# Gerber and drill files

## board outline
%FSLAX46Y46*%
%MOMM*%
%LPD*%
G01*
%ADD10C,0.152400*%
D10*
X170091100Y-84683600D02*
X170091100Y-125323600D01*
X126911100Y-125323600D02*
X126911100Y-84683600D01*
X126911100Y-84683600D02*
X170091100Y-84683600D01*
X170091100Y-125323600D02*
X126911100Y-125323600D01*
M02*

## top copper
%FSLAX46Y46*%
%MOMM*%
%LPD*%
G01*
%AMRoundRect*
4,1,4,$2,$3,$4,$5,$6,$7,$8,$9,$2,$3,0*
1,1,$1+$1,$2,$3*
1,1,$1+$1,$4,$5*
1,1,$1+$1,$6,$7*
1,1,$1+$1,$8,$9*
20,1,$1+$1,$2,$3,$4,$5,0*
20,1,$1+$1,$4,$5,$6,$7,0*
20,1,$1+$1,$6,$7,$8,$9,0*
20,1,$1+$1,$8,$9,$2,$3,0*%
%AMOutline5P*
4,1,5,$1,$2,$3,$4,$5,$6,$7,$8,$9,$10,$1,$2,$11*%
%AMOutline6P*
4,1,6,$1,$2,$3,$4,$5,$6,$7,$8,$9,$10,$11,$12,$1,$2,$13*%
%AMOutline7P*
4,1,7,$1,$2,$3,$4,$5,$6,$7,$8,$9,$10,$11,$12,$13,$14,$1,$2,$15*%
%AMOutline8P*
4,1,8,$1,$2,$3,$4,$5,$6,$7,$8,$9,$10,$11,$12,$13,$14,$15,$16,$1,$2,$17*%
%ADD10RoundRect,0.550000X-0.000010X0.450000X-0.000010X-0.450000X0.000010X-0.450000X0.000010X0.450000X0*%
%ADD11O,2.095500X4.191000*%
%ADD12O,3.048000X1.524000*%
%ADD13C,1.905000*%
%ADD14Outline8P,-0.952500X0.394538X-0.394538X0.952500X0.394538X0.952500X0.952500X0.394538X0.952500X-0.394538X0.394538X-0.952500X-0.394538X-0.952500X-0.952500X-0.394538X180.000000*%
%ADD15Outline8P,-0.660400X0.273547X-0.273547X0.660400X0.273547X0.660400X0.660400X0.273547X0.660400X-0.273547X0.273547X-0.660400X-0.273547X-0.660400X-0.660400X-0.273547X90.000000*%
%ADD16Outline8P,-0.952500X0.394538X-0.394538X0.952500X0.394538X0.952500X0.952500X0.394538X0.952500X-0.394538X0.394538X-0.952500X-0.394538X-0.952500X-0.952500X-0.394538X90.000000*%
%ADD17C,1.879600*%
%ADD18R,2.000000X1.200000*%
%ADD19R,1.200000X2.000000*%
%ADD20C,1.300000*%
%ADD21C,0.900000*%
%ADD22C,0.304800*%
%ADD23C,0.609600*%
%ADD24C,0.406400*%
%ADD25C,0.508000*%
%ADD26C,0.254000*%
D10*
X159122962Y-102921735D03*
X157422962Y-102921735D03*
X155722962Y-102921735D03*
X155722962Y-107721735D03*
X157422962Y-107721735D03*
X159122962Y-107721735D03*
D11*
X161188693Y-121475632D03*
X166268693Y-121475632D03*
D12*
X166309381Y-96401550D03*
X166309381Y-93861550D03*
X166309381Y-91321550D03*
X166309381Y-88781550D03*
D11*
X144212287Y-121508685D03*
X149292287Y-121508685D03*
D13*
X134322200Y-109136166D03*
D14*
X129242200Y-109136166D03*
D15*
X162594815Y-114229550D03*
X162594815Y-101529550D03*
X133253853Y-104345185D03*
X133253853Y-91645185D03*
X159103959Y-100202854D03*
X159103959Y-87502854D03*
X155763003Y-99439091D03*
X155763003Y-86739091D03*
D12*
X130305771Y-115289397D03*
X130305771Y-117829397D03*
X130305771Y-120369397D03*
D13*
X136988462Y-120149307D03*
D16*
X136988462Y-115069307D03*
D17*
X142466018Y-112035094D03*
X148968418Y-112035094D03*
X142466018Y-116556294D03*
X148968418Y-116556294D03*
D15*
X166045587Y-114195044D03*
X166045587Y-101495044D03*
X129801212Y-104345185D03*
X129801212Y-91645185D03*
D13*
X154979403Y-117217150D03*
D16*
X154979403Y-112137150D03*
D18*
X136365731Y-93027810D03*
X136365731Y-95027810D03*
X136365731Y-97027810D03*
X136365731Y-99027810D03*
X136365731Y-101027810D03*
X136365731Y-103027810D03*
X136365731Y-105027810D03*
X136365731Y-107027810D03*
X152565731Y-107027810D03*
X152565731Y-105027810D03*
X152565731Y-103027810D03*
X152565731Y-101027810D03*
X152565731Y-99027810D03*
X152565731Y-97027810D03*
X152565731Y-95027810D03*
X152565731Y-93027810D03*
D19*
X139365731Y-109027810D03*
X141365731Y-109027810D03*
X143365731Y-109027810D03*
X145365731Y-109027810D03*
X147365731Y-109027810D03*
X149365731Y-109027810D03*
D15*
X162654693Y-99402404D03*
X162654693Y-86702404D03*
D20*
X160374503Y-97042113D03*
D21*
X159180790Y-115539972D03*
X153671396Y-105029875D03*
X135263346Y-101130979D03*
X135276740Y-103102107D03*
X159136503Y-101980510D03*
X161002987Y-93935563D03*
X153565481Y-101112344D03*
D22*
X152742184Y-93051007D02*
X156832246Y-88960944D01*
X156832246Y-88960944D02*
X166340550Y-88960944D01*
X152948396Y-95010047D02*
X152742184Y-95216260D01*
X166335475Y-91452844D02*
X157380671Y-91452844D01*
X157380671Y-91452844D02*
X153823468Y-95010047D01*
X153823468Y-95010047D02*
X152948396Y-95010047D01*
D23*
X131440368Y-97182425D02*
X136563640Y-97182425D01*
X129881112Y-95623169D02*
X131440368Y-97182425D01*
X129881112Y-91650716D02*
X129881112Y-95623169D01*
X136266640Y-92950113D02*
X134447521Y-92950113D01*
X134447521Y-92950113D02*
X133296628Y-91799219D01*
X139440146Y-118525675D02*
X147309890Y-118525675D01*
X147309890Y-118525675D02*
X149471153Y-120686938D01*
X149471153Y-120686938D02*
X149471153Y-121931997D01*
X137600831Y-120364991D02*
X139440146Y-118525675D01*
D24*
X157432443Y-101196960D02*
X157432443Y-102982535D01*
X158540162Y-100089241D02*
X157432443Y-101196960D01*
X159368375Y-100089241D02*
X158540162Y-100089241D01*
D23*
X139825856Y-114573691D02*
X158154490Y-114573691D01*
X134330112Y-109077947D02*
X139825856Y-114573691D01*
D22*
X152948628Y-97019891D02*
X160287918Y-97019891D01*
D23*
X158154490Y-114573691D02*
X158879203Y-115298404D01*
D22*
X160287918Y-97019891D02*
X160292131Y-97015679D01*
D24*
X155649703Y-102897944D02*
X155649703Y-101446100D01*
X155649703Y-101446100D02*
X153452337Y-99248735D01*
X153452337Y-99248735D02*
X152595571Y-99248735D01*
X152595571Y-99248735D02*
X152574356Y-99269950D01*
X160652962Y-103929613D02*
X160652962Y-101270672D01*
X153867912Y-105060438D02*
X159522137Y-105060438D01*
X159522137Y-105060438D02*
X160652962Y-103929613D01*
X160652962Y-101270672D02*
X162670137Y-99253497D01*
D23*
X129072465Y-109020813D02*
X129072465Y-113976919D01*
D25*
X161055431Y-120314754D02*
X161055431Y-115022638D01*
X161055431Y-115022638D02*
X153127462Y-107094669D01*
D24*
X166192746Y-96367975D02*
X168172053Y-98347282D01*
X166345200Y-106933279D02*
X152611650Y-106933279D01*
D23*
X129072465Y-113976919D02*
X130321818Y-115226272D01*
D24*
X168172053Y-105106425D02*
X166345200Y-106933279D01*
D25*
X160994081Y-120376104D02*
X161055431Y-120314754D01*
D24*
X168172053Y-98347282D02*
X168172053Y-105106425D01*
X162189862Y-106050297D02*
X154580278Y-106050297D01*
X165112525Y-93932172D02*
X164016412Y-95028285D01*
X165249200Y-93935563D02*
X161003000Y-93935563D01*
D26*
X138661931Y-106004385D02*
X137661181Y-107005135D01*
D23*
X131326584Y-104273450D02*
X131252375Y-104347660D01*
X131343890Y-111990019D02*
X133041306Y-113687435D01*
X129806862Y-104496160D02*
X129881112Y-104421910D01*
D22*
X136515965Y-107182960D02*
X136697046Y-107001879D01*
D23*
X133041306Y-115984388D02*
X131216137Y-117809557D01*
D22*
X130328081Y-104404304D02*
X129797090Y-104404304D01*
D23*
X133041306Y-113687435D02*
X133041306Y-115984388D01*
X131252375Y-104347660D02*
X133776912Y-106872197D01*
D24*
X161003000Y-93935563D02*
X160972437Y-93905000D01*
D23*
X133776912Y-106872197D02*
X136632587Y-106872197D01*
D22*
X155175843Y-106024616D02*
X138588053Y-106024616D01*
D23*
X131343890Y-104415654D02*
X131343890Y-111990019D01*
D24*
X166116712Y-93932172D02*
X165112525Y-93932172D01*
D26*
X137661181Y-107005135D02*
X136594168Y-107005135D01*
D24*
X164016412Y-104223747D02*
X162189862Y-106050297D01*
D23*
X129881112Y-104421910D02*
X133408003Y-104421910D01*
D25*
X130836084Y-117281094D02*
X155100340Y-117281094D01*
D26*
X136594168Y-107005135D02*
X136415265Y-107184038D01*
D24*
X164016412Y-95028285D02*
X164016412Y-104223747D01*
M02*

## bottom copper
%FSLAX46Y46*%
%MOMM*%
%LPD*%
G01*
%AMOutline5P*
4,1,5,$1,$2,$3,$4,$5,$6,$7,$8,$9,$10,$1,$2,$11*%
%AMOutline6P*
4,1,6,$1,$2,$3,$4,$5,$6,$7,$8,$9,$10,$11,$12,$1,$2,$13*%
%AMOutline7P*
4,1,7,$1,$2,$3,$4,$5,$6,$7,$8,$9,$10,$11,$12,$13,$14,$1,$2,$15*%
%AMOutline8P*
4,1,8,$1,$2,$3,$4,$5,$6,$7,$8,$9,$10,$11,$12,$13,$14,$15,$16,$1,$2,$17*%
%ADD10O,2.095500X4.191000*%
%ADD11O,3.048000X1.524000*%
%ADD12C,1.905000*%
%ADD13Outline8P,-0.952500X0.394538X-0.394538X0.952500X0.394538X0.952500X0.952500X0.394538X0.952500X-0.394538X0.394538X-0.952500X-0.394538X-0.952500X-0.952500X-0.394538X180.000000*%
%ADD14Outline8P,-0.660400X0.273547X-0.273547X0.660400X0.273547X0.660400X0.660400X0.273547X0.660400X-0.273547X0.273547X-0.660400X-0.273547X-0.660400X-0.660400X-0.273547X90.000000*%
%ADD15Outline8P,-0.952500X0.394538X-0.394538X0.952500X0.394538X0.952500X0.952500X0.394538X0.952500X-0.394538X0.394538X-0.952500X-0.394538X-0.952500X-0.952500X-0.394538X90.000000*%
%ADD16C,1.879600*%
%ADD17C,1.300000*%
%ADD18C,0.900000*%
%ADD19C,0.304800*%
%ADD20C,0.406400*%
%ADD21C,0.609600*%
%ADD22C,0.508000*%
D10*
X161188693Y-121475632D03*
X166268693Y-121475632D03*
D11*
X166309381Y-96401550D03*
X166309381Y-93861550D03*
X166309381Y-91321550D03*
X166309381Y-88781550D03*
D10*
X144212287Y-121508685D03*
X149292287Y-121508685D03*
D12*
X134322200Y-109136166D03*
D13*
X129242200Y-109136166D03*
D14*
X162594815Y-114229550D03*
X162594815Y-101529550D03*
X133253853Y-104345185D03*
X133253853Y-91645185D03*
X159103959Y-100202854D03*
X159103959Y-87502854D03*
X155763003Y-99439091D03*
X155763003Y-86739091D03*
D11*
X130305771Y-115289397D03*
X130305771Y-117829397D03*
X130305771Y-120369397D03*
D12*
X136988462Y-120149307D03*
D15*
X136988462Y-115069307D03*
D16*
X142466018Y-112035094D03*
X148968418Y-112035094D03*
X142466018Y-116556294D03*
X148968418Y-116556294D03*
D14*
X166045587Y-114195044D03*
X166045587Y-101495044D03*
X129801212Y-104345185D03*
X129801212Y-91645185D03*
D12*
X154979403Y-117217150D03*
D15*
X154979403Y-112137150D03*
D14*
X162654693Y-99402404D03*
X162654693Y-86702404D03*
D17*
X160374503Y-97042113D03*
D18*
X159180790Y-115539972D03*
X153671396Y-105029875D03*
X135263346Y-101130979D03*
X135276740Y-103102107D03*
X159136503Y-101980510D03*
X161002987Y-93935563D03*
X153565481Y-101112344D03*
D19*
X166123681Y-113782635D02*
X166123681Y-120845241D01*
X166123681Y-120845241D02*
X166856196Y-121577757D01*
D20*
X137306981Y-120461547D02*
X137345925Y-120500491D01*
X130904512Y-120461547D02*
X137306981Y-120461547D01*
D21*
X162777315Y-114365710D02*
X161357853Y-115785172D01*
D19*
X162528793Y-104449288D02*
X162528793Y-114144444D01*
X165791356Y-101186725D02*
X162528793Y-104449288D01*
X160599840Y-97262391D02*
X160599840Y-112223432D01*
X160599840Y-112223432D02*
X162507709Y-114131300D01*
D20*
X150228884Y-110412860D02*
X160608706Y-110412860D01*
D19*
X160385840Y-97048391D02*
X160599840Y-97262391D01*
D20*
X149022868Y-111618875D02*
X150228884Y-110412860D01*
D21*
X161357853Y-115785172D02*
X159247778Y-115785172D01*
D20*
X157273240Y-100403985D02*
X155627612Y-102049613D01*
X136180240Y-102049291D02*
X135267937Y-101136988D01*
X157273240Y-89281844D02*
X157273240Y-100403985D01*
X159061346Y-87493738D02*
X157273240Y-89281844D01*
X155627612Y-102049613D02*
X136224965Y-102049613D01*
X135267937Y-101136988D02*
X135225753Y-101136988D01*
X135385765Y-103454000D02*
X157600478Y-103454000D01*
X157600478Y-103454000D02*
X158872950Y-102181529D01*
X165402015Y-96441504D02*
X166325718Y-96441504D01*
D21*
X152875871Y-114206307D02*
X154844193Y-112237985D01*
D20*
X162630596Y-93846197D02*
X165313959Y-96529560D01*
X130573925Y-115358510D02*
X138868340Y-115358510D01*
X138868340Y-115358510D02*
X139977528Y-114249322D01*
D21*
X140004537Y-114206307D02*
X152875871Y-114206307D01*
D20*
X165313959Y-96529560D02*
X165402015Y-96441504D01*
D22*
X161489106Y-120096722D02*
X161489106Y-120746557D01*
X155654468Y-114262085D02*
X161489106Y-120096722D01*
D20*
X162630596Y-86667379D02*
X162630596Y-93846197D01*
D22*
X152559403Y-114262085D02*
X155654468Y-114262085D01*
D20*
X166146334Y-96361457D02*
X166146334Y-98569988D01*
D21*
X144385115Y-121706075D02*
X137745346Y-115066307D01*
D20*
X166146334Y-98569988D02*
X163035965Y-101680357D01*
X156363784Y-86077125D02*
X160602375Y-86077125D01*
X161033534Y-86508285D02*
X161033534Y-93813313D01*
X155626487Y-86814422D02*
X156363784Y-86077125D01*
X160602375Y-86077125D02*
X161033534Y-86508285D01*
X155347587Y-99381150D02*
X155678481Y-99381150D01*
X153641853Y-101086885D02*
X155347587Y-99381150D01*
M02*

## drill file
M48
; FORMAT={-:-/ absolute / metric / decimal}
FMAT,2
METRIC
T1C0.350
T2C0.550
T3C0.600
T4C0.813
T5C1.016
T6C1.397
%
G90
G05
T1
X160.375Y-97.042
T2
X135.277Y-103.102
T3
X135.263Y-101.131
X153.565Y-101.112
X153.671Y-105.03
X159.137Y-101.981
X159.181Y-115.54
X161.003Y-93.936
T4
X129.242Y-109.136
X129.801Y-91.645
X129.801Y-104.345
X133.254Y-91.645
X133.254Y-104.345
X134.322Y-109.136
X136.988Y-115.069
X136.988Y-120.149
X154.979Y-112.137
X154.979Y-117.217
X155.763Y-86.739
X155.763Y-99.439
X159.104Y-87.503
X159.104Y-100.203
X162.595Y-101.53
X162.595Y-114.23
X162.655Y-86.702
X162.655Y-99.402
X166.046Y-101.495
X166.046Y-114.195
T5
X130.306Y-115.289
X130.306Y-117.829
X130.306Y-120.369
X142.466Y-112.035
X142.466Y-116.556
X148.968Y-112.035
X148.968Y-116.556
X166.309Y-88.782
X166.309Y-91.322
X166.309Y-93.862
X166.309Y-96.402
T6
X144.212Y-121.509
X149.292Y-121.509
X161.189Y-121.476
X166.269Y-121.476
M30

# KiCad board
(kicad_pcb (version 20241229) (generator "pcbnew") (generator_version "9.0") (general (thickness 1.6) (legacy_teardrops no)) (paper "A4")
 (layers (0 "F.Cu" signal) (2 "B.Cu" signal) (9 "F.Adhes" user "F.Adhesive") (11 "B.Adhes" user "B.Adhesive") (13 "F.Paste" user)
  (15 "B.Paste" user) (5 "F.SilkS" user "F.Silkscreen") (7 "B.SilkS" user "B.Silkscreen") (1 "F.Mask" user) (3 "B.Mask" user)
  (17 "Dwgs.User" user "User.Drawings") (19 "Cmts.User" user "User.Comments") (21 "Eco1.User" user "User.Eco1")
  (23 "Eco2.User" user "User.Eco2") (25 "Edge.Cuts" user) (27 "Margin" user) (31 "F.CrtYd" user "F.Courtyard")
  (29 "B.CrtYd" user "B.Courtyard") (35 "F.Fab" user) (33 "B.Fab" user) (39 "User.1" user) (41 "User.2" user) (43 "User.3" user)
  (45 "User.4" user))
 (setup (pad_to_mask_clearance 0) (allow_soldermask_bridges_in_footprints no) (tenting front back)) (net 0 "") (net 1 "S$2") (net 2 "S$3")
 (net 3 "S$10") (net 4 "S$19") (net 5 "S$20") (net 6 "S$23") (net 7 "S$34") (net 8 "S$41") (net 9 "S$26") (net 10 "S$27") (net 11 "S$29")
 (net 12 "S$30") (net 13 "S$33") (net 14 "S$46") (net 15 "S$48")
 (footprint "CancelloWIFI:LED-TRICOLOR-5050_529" (layer "F.Cu") (at 157.422962 105.321735 -90)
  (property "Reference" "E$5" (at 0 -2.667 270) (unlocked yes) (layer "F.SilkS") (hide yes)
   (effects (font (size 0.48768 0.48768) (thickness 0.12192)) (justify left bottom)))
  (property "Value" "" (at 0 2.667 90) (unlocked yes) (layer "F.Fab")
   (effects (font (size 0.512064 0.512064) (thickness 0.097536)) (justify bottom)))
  (pad "1" smd roundrect (at -2.4 -1.7 270) (size 2 1.1) (layers "F.Cu" "F.Mask" "F.Paste") (roundrect_rratio 0.5)
   (solder_mask_margin 0.1016) (solder_paste_margin 0) (thermal_bridge_angle 0))
  (pad "2" smd roundrect (at -2.4 0 270) (size 2 1.1) (layers "F.Cu" "F.Mask" "F.Paste") (roundrect_rratio 0.5) (solder_mask_margin 0.1016)
   (solder_paste_margin 0) (thermal_bridge_angle 0))
  (pad "3" smd roundrect (at -2.4 1.7 270) (size 2 1.1) (layers "F.Cu" "F.Mask" "F.Paste") (roundrect_rratio 0.5)
   (solder_mask_margin 0.1016) (solder_paste_margin 0) (thermal_bridge_angle 0))
  (pad "4" smd roundrect (at 2.4 1.7 270) (size 2 1.1) (layers "F.Cu" "F.Mask" "F.Paste") (roundrect_rratio 0.5) (solder_mask_margin 0.1016)
   (solder_paste_margin 0) (thermal_bridge_angle 0))
  (pad "5" smd roundrect (at 2.4 0 270) (size 2 1.1) (layers "F.Cu" "F.Mask" "F.Paste") (roundrect_rratio 0.5) (solder_mask_margin 0.1016)
   (solder_paste_margin 0) (thermal_bridge_angle 0))
  (pad "6" smd roundrect (at 2.4 -1.7 270) (size 2 1.1) (layers "F.Cu" "F.Mask" "F.Paste") (roundrect_rratio 0.5)
   (solder_mask_margin 0.1016) (solder_paste_margin 0) (thermal_bridge_angle 0)))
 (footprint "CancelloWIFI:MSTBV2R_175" (layer "F.Cu") (at 163.728693 121.475632)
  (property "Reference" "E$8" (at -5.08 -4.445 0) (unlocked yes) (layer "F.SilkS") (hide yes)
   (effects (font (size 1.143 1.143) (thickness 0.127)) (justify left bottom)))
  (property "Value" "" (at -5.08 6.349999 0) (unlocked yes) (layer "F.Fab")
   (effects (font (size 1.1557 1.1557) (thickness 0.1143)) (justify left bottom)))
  (pad "1" thru_hole oval (at -2.54 0 90) (size 4.191 2.0955) (drill 1.397) (layers "*.Cu" "*.Mask") (remove_unused_layers no)
   (solder_mask_margin 0.1016) (thermal_bridge_angle 0))
  (pad "2" thru_hole oval (at 2.54 0 90) (size 4.191 2.0955) (drill 1.397) (layers "*.Cu" "*.Mask") (remove_unused_layers no)
   (solder_mask_margin 0.1016) (thermal_bridge_angle 0)))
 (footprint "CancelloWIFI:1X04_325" (layer "F.Cu") (at 166.309381 92.59155 90)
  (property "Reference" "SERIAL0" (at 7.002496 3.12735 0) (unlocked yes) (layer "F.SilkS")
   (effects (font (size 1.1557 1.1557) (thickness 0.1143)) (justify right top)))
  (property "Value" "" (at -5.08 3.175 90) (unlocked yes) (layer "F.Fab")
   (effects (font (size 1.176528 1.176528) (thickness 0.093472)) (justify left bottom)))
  (pad "1" thru_hole oval (at -3.81 0 180) (size 3.048 1.524) (drill 1.016) (layers "*.Cu" "*.Mask") (remove_unused_layers no)
   (solder_mask_margin 0.1016) (thermal_bridge_angle 0))
  (pad "2" thru_hole oval (at -1.27 0 180) (size 3.048 1.524) (drill 1.016) (layers "*.Cu" "*.Mask") (remove_unused_layers no)
   (solder_mask_margin 0.1016) (thermal_bridge_angle 0))
  (pad "3" thru_hole oval (at 1.27 0 180) (size 3.048 1.524) (drill 1.016) (layers "*.Cu" "*.Mask") (remove_unused_layers no)
   (solder_mask_margin 0.1016) (thermal_bridge_angle 0))
  (pad "4" thru_hole oval (at 3.81 0 180) (size 3.048 1.524) (drill 1.016) (layers "*.Cu" "*.Mask") (remove_unused_layers no)
   (solder_mask_margin 0.1016) (thermal_bridge_angle 0)))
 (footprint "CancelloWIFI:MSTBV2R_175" (layer "F.Cu") (at 146.752287 121.508685)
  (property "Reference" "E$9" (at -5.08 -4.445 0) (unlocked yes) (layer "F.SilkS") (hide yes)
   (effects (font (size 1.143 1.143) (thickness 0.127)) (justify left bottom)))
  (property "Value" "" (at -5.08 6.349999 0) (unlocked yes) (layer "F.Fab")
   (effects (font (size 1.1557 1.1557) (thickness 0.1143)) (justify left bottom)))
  (pad "1" thru_hole oval (at -2.54 0 90) (size 4.191 2.0955) (drill 1.397) (layers "*.Cu" "*.Mask") (remove_unused_layers no)
   (solder_mask_margin 0.1016) (thermal_bridge_angle 0))
  (pad "2" thru_hole oval (at 2.54 0 90) (size 4.191 2.0955) (drill 1.397) (layers "*.Cu" "*.Mask") (remove_unused_layers no)
   (solder_mask_margin 0.1016) (thermal_bridge_angle 0)))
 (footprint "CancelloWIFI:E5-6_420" (layer "F.Cu") (at 131.7822 109.136166 180)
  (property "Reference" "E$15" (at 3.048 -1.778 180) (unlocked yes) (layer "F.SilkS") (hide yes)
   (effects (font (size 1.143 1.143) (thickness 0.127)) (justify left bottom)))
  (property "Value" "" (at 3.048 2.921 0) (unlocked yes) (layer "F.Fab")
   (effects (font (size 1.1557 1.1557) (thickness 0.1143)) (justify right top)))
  (pad "+" thru_hole circle (at -2.54 0 180) (size 1.905 1.905) (drill 0.8128) (layers "*.Cu" "*.Mask") (remove_unused_layers no)
   (solder_mask_margin 0.1016) (thermal_bridge_angle 0))
  (pad "-" thru_hole roundrect (at 2.54 0 180) (size 1.905 1.905) (drill 0.8128) (layers "*.Cu" "*.Mask") (remove_unused_layers no)
   (roundrect_rratio 0.25) (chamfer_ratio 0.2928932188) (chamfer top_left top_right bottom_left bottom_right) (solder_mask_margin 0.1016)
   (thermal_bridge_angle 0)))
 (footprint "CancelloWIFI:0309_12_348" (layer "F.Cu") (at 162.594815 107.87955 90)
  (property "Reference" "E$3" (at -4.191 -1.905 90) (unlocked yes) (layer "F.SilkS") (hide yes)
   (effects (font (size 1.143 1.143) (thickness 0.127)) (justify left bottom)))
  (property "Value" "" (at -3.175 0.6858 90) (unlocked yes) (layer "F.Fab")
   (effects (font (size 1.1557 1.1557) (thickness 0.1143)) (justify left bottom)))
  (pad "1" thru_hole roundrect (at -6.35 0 90) (size 1.3208 1.3208) (drill 0.8128) (layers "*.Cu" "*.Mask") (remove_unused_layers no)
   (roundrect_rratio 0.25) (chamfer_ratio 0.2928932188) (chamfer top_left top_right bottom_left bottom_right) (solder_mask_margin 0.1016)
   (thermal_bridge_angle 0))
  (pad "2" thru_hole roundrect (at 6.35 0 90) (size 1.3208 1.3208) (drill 0.8128) (layers "*.Cu" "*.Mask") (remove_unused_layers no)
   (roundrect_rratio 0.25) (chamfer_ratio 0.2928932188) (chamfer top_left top_right bottom_left bottom_right) (solder_mask_margin 0.1016)
   (thermal_bridge_angle 0)))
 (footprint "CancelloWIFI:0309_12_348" (layer "F.Cu") (at 133.253853 97.995185 90)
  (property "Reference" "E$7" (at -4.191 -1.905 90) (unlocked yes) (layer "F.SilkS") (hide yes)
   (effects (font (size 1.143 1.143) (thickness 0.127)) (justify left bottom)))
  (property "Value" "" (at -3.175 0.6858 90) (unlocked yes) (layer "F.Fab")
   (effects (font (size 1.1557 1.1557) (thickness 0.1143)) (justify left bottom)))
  (pad "1" thru_hole roundrect (at -6.35 0 90) (size 1.3208 1.3208) (drill 0.8128) (layers "*.Cu" "*.Mask") (remove_unused_layers no)
   (roundrect_rratio 0.25) (chamfer_ratio 0.2928932188) (chamfer top_left top_right bottom_left bottom_right) (solder_mask_margin 0.1016)
   (thermal_bridge_angle 0))
  (pad "2" thru_hole roundrect (at 6.35 0 90) (size 1.3208 1.3208) (drill 0.8128) (layers "*.Cu" "*.Mask") (remove_unused_layers no)
   (roundrect_rratio 0.25) (chamfer_ratio 0.2928932188) (chamfer top_left top_right bottom_left bottom_right) (solder_mask_margin 0.1016)
   (thermal_bridge_angle 0)))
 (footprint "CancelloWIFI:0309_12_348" (layer "F.Cu") (at 159.103959 93.852854 90)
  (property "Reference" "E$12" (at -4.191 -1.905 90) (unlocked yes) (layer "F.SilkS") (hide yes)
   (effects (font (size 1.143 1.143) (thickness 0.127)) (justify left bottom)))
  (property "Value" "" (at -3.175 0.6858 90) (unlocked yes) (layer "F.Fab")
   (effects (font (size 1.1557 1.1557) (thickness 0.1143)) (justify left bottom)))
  (pad "1" thru_hole roundrect (at -6.35 0 90) (size 1.3208 1.3208) (drill 0.8128) (layers "*.Cu" "*.Mask") (remove_unused_layers no)
   (roundrect_rratio 0.25) (chamfer_ratio 0.2928932188) (chamfer top_left top_right bottom_left bottom_right) (solder_mask_margin 0.1016)
   (thermal_bridge_angle 0))
  (pad "2" thru_hole roundrect (at 6.35 0 90) (size 1.3208 1.3208) (drill 0.8128) (layers "*.Cu" "*.Mask") (remove_unused_layers no)
   (roundrect_rratio 0.25) (chamfer_ratio 0.2928932188) (chamfer top_left top_right bottom_left bottom_right) (solder_mask_margin 0.1016)
   (thermal_bridge_angle 0)))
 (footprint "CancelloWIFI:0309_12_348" (layer "F.Cu") (at 155.763003 93.089091 90)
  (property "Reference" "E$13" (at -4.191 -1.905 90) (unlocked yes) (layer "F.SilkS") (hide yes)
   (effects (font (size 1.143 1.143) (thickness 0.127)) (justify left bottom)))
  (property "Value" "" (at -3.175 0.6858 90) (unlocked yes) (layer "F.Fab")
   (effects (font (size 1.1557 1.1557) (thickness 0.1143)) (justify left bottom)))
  (pad "1" thru_hole roundrect (at -6.35 0 90) (size 1.3208 1.3208) (drill 0.8128) (layers "*.Cu" "*.Mask") (remove_unused_layers no)
   (roundrect_rratio 0.25) (chamfer_ratio 0.2928932188) (chamfer top_left top_right bottom_left bottom_right) (solder_mask_margin 0.1016)
   (thermal_bridge_angle 0))
  (pad "2" thru_hole roundrect (at 6.35 0 90) (size 1.3208 1.3208) (drill 0.8128) (layers "*.Cu" "*.Mask") (remove_unused_layers no)
   (roundrect_rratio 0.25) (chamfer_ratio 0.2928932188) (chamfer top_left top_right bottom_left bottom_right) (solder_mask_margin 0.1016)
   (thermal_bridge_angle 0)))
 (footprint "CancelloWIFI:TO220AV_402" (layer "F.Cu") (at 132.845771 117.829397 -90)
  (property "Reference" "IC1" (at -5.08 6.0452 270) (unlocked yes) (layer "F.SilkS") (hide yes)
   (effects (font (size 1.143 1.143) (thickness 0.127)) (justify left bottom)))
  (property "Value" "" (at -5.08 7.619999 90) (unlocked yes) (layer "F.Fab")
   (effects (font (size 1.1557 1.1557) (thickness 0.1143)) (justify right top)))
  (pad "1" thru_hole oval (at -2.54 2.54) (size 3.048 1.524) (drill 1.016) (layers "*.Cu" "*.Mask") (remove_unused_layers no)
   (solder_mask_margin 0.1016) (thermal_bridge_angle 0))
  (pad "2" thru_hole oval (at 0 2.54) (size 3.048 1.524) (drill 1.016) (layers "*.Cu" "*.Mask") (remove_unused_layers no)
   (solder_mask_margin 0.1016) (thermal_bridge_angle 0))
  (pad "3" thru_hole oval (at 2.54 2.54) (size 3.048 1.524) (drill 1.016) (layers "*.Cu" "*.Mask") (remove_unused_layers no)
   (solder_mask_margin 0.1016) (thermal_bridge_angle 0)))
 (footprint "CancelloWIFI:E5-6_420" (layer "F.Cu") (at 136.988462 117.609307 90)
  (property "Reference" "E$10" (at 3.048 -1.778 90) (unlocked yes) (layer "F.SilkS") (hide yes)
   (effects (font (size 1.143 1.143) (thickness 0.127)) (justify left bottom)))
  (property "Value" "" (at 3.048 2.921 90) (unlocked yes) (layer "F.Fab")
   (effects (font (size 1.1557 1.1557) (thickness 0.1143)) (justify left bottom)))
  (pad "+" thru_hole circle (at -2.54 0 90) (size 1.905 1.905) (drill 0.8128) (layers "*.Cu" "*.Mask") (remove_unused_layers no)
   (solder_mask_margin 0.1016) (thermal_bridge_angle 0))
  (pad "-" thru_hole roundrect (at 2.54 0 90) (size 1.905 1.905) (drill 0.8128) (layers "*.Cu" "*.Mask") (remove_unused_layers no)
   (roundrect_rratio 0.25) (chamfer_ratio 0.2928932188) (chamfer top_left top_right bottom_left bottom_right) (solder_mask_margin 0.1016)
   (thermal_bridge_angle 0)))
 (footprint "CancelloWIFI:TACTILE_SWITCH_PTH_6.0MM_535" (layer "F.Cu") (at 145.717218 114.295694)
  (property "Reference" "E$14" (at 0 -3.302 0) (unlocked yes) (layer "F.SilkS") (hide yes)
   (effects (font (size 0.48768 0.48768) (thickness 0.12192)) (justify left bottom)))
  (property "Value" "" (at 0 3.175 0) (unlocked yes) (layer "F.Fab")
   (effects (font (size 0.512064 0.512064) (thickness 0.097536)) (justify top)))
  (pad "1" thru_hole circle (at -3.2512 -2.2606) (size 1.8796 1.8796) (drill 1.016) (layers "*.Cu" "*.Mask") (remove_unused_layers no)
   (solder_mask_margin 0.1016) (thermal_bridge_angle 0))
  (pad "2" thru_hole circle (at 3.2512 -2.2606) (size 1.8796 1.8796) (drill 1.016) (layers "*.Cu" "*.Mask") (remove_unused_layers no)
   (solder_mask_margin 0.1016) (thermal_bridge_angle 0))
  (pad "3" thru_hole circle (at -3.2512 2.2606) (size 1.8796 1.8796) (drill 1.016) (layers "*.Cu" "*.Mask") (remove_unused_layers no)
   (solder_mask_margin 0.1016) (thermal_bridge_angle 0))
  (pad "4" thru_hole circle (at 3.2512 2.2606) (size 1.8796 1.8796) (drill 1.016) (layers "*.Cu" "*.Mask") (remove_unused_layers no)
   (solder_mask_margin 0.1016) (thermal_bridge_angle 0)))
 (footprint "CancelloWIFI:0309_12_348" (layer "F.Cu") (at 166.045587 107.845044 90)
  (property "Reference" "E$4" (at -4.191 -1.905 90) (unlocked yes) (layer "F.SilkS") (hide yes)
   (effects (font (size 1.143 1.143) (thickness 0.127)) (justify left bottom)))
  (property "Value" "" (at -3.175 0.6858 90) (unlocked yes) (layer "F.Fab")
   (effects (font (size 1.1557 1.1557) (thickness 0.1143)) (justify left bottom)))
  (pad "1" thru_hole roundrect (at -6.35 0 90) (size 1.3208 1.3208) (drill 0.8128) (layers "*.Cu" "*.Mask") (remove_unused_layers no)
   (roundrect_rratio 0.25) (chamfer_ratio 0.2928932188) (chamfer top_left top_right bottom_left bottom_right) (solder_mask_margin 0.1016)
   (thermal_bridge_angle 0))
  (pad "2" thru_hole roundrect (at 6.35 0 90) (size 1.3208 1.3208) (drill 0.8128) (layers "*.Cu" "*.Mask") (remove_unused_layers no)
   (roundrect_rratio 0.25) (chamfer_ratio 0.2928932188) (chamfer top_left top_right bottom_left bottom_right) (solder_mask_margin 0.1016)
   (thermal_bridge_angle 0)))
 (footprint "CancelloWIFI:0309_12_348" (layer "F.Cu") (at 129.801212 97.995185 90)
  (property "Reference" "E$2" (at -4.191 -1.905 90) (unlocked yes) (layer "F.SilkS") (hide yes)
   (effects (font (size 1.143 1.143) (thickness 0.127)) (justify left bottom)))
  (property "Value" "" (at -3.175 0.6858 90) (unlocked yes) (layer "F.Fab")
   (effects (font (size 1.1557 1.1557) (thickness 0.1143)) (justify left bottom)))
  (pad "1" thru_hole roundrect (at -6.35 0 90) (size 1.3208 1.3208) (drill 0.8128) (layers "*.Cu" "*.Mask") (remove_unused_layers no)
   (roundrect_rratio 0.25) (chamfer_ratio 0.2928932188) (chamfer top_left top_right bottom_left bottom_right) (solder_mask_margin 0.1016)
   (thermal_bridge_angle 0))
  (pad "2" thru_hole roundrect (at 6.35 0 90) (size 1.3208 1.3208) (drill 0.8128) (layers "*.Cu" "*.Mask") (remove_unused_layers no)
   (roundrect_rratio 0.25) (chamfer_ratio 0.2928932188) (chamfer top_left top_right bottom_left bottom_right) (solder_mask_margin 0.1016)
   (thermal_bridge_angle 0)))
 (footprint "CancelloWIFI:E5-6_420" (layer "F.Cu") (at 154.979403 114.67715 90)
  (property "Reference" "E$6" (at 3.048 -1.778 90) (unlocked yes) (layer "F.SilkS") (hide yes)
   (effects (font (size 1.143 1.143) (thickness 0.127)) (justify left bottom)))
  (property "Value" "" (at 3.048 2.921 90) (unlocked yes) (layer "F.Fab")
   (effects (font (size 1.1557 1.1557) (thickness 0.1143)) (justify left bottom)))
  (pad "+" thru_hole circle (at -2.54 0 90) (size 1.905 1.905) (drill 0.8128) (layers "*.Cu" "*.Mask") (remove_unused_layers no)
   (solder_mask_margin 0.1016) (thermal_bridge_angle 0))
  (pad "-" thru_hole roundrect (at 2.54 0 90) (size 1.905 1.905) (drill 0.8128) (layers "*.Cu" "*.Mask") (remove_unused_layers no)
   (roundrect_rratio 0.25) (chamfer_ratio 0.2928932188) (chamfer top_left top_right bottom_left bottom_right) (solder_mask_margin 0.1016)
   (thermal_bridge_angle 0)))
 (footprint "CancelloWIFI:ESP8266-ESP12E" (layer "F.Cu") (at 143.985731 98.86781)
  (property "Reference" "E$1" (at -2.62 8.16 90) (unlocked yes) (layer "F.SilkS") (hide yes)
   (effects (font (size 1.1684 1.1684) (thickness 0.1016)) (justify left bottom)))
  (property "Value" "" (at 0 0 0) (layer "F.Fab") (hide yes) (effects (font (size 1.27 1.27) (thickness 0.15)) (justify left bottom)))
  (pad "1" smd rect (at -7.62 -5.84) (size 2 1.2) (layers "F.Cu" "F.Mask" "F.Paste") (solder_mask_margin 0.1016) (solder_paste_margin 0)
   (thermal_bridge_angle 0))
  (pad "2" smd rect (at -7.62 -3.84) (size 2 1.2) (layers "F.Cu" "F.Mask" "F.Paste") (solder_mask_margin 0.1016) (solder_paste_margin 0)
   (thermal_bridge_angle 0))
  (pad "3" smd rect (at -7.62 -1.84) (size 2 1.2) (layers "F.Cu" "F.Mask" "F.Paste") (solder_mask_margin 0.1016) (solder_paste_margin 0)
   (thermal_bridge_angle 0))
  (pad "4" smd rect (at -7.62 0.16) (size 2 1.2) (layers "F.Cu" "F.Mask" "F.Paste") (solder_mask_margin 0.1016) (solder_paste_margin 0)
   (thermal_bridge_angle 0))
  (pad "5" smd rect (at -7.62 2.16) (size 2 1.2) (layers "F.Cu" "F.Mask" "F.Paste") (solder_mask_margin 0.1016) (solder_paste_margin 0)
   (thermal_bridge_angle 0))
  (pad "6" smd rect (at -7.62 4.16) (size 2 1.2) (layers "F.Cu" "F.Mask" "F.Paste") (solder_mask_margin 0.1016) (solder_paste_margin 0)
   (thermal_bridge_angle 0))
  (pad "7" smd rect (at -7.62 6.16) (size 2 1.2) (layers "F.Cu" "F.Mask" "F.Paste") (solder_mask_margin 0.1016) (solder_paste_margin 0)
   (thermal_bridge_angle 0))
  (pad "8" smd rect (at -7.62 8.16) (size 2 1.2) (layers "F.Cu" "F.Mask" "F.Paste") (solder_mask_margin 0.1016) (solder_paste_margin 0)
   (thermal_bridge_angle 0))
  (pad "9" smd rect (at 8.58 8.16) (size 2 1.2) (layers "F.Cu" "F.Mask" "F.Paste") (solder_mask_margin 0.1016) (solder_paste_margin 0)
   (thermal_bridge_angle 0))
  (pad "10" smd rect (at 8.58 6.16) (size 2 1.2) (layers "F.Cu" "F.Mask" "F.Paste") (solder_mask_margin 0.1016) (solder_paste_margin 0)
   (thermal_bridge_angle 0))
  (pad "11" smd rect (at 8.58 4.16) (size 2 1.2) (layers "F.Cu" "F.Mask" "F.Paste") (solder_mask_margin 0.1016) (solder_paste_margin 0)
   (thermal_bridge_angle 0))
  (pad "12" smd rect (at 8.58 2.16) (size 2 1.2) (layers "F.Cu" "F.Mask" "F.Paste") (solder_mask_margin 0.1016) (solder_paste_margin 0)
   (thermal_bridge_angle 0))
  (pad "13" smd rect (at 8.58 0.16) (size 2 1.2) (layers "F.Cu" "F.Mask" "F.Paste") (solder_mask_margin 0.1016) (solder_paste_margin 0)
   (thermal_bridge_angle 0))
  (pad "14" smd rect (at 8.58 -1.84) (size 2 1.2) (layers "F.Cu" "F.Mask" "F.Paste") (solder_mask_margin 0.1016) (solder_paste_margin 0)
   (thermal_bridge_angle 0))
  (pad "15" smd rect (at 8.58 -3.84) (size 2 1.2) (layers "F.Cu" "F.Mask" "F.Paste") (solder_mask_margin 0.1016) (solder_paste_margin 0)
   (thermal_bridge_angle 0))
  (pad "16" smd rect (at 8.58 -5.84) (size 2 1.2) (layers "F.Cu" "F.Mask" "F.Paste") (solder_mask_margin 0.1016) (solder_paste_margin 0)
   (thermal_bridge_angle 0))
  (pad "17" smd rect (at -4.62 10.16 90) (size 2 1.2) (layers "F.Cu" "F.Mask" "F.Paste") (solder_mask_margin 0.1016) (solder_paste_margin 0)
   (thermal_bridge_angle 0))
  (pad "18" smd rect (at -2.62 10.16 90) (size 2 1.2) (layers "F.Cu" "F.Mask" "F.Paste") (solder_mask_margin 0.1016) (solder_paste_margin 0)
   (thermal_bridge_angle 0))
  (pad "19" smd rect (at -0.62 10.16 90) (size 2 1.2) (layers "F.Cu" "F.Mask" "F.Paste") (solder_mask_margin 0.1016) (solder_paste_margin 0)
   (thermal_bridge_angle 0))
  (pad "20" smd rect (at 1.38 10.16 90) (size 2 1.2) (layers "F.Cu" "F.Mask" "F.Paste") (solder_mask_margin 0.1016) (solder_paste_margin 0)
   (thermal_bridge_angle 0))
  (pad "21" smd rect (at 3.38 10.16 90) (size 2 1.2) (layers "F.Cu" "F.Mask" "F.Paste") (solder_mask_margin 0.1016) (solder_paste_margin 0)
   (thermal_bridge_angle 0))
  (pad "22" smd rect (at 5.38 10.16 90) (size 2 1.2) (layers "F.Cu" "F.Mask" "F.Paste") (solder_mask_margin 0.1016) (solder_paste_margin 0)
   (thermal_bridge_angle 0))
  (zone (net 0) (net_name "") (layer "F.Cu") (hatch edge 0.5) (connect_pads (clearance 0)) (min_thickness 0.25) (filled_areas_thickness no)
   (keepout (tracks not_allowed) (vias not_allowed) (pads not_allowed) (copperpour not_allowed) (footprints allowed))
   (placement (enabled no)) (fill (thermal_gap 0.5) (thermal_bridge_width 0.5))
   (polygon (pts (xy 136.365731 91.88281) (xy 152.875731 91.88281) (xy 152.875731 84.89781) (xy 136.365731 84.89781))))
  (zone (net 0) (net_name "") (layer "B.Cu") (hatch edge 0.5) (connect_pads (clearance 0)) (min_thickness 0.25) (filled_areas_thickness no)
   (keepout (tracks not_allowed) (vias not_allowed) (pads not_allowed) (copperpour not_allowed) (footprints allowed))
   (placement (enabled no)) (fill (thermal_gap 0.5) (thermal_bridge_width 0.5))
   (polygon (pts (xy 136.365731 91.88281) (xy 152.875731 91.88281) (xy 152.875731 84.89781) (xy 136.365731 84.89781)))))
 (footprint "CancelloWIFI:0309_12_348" (layer "F.Cu") (at 162.654693 93.052404 90)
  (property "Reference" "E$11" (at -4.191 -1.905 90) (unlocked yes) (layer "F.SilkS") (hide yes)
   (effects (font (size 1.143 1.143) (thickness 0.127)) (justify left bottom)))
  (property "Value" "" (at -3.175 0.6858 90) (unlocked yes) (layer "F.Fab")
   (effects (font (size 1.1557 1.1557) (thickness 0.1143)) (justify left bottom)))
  (pad "1" thru_hole roundrect (at -6.35 0 90) (size 1.3208 1.3208) (drill 0.8128) (layers "*.Cu" "*.Mask") (remove_unused_layers no)
   (roundrect_rratio 0.25) (chamfer_ratio 0.2928932188) (chamfer top_left top_right bottom_left bottom_right) (solder_mask_margin 0.1016)
   (thermal_bridge_angle 0))
  (pad "2" thru_hole roundrect (at 6.35 0 90) (size 1.3208 1.3208) (drill 0.8128) (layers "*.Cu" "*.Mask") (remove_unused_layers no)
   (roundrect_rratio 0.25) (chamfer_ratio 0.2928932188) (chamfer top_left top_right bottom_left bottom_right) (solder_mask_margin 0.1016)
   (thermal_bridge_angle 0)))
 (gr_line (start 170.0911 84.6836) (end 170.0911 125.3236) (stroke (width 0.1524) (type solid)) (layer "Edge.Cuts"))
 (gr_line (start 126.9111 125.3236) (end 126.9111 84.6836) (stroke (width 0.1524) (type solid)) (layer "Edge.Cuts"))
 (gr_line (start 126.9111 84.6836) (end 170.0911 84.6836) (stroke (width 0.1524) (type solid)) (layer "Edge.Cuts"))
 (gr_line (start 170.0911 125.3236) (end 126.9111 125.3236) (stroke (width 0.1524) (type solid)) (layer "Edge.Cuts"))
 (segment (start 152.742184 93.051007) (end 156.832246 88.960944) (width 0.3048) (layer "F.Cu") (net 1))
 (segment (start 156.832246 88.960944) (end 166.34055 88.960944) (width 0.3048) (layer "F.Cu") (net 1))
 (segment (start 152.948396 95.010047) (end 152.742184 95.21626) (width 0.3048) (layer "F.Cu") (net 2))
 (segment (start 166.335475 91.452844) (end 157.380671 91.452844) (width 0.3048) (layer "F.Cu") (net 2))
 (segment (start 157.380671 91.452844) (end 153.823468 95.010047) (width 0.3048) (layer "F.Cu") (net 2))
 (segment (start 153.823468 95.010047) (end 152.948396 95.010047) (width 0.3048) (layer "F.Cu") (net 2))
 (segment (start 166.123681 113.782635) (end 166.123681 120.845241) (width 0.3048) (layer "B.Cu") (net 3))
 (segment (start 166.123681 120.845241) (end 166.856196 121.577757) (width 0.3048) (layer "B.Cu") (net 3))
 (segment (start 131.440368 97.182425) (end 136.56364 97.182425) (width 0.6096) (layer "F.Cu") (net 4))
 (segment (start 129.881112 95.623169) (end 131.440368 97.182425) (width 0.6096) (layer "F.Cu") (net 4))
 (segment (start 129.881112 91.650716) (end 129.881112 95.623169) (width 0.6096) (layer "F.Cu") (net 4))
 (segment (start 136.26664 92.950113) (end 134.447521 92.950113) (width 0.6096) (layer "F.Cu") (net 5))
 (segment (start 134.447521 92.950113) (end 133.296628 91.799219) (width 0.6096) (layer "F.Cu") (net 5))
 (segment (start 139.440146 118.525675) (end 147.30989 118.525675) (width 0.6096) (layer "F.Cu") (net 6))
 (segment (start 147.30989 118.525675) (end 149.471153 120.686938) (width 0.6096) (layer "F.Cu") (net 6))
 (segment (start 149.471153 120.686938) (end 149.471153 121.931997) (width 0.6096) (layer "F.Cu") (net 6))
 (segment (start 137.600831 120.364991) (end 139.440146 118.525675) (width 0.6096) (layer "F.Cu") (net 6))
 (segment (start 137.306981 120.461547) (end 137.345925 120.500491) (width 0.4064) (layer "B.Cu") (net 6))
 (segment (start 130.904512 120.461547) (end 137.306981 120.461547) (width 0.4064) (layer "B.Cu") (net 6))
 (segment (start 157.432443 101.19696) (end 157.432443 102.982535) (width 0.4064) (layer "F.Cu") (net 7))
 (segment (start 158.540162 100.089241) (end 157.432443 101.19696) (width 0.4064) (layer "F.Cu") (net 7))
 (segment (start 159.368375 100.089241) (end 158.540162 100.089241) (width 0.4064) (layer "F.Cu") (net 7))
 (segment (start 139.825856 114.573691) (end 158.15449 114.573691) (width 0.6096) (layer "F.Cu") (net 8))
 (segment (start 134.330112 109.077947) (end 139.825856 114.573691) (width 0.6096) (layer "F.Cu") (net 8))
 (segment (start 152.948628 97.019891) (end 160.287918 97.019891) (width 0.3048) (layer "F.Cu") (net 8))
 (segment (start 158.15449 114.573691) (end 158.879203 115.298404) (width 0.6096) (layer "F.Cu") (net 8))
 (segment (start 160.287918 97.019891) (end 160.292131 97.015679) (width 0.3048) (layer "F.Cu") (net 8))
 (via (at 160.374503 97.042113) (size 1.3) (drill 0.35) (layers "F.Cu" "B.Cu") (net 8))
 (via (at 159.18079 115.539972) (size 0.9) (drill 0.6) (layers "F.Cu" "B.Cu") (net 8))
 (segment (start 162.777315 114.36571) (end 161.357853 115.785172) (width 0.6096) (layer "B.Cu") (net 8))
 (segment (start 162.528793 104.449288) (end 162.528793 114.144444) (width 0.3048) (layer "B.Cu") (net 8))
 (segment (start 165.791356 101.186725) (end 162.528793 104.449288) (width 0.3048) (layer "B.Cu") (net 8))
 (segment (start 160.59984 97.262391) (end 160.59984 112.223432) (width 0.3048) (layer "B.Cu") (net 8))
 (segment (start 160.59984 112.223432) (end 162.507709 114.1313) (width 0.3048) (layer "B.Cu") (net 8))
 (segment (start 150.228884 110.41286) (end 160.608706 110.41286) (width 0.4064) (layer "B.Cu") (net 8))
 (segment (start 160.38584 97.048391) (end 160.59984 97.262391) (width 0.3048) (layer "B.Cu") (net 8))
 (segment (start 149.022868 111.618875) (end 150.228884 110.41286) (width 0.4064) (layer "B.Cu") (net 8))
 (segment (start 161.357853 115.785172) (end 159.247778 115.785172) (width 0.6096) (layer "B.Cu") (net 8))
 (segment (start 155.649703 102.897944) (end 155.649703 101.4461) (width 0.4064) (layer "F.Cu") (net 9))
 (segment (start 155.649703 101.4461) (end 153.452337 99.248735) (width 0.4064) (layer "F.Cu") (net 9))
 (segment (start 153.452337 99.248735) (end 152.595571 99.248735) (width 0.4064) (layer "F.Cu") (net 9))
 (segment (start 152.595571 99.248735) (end 152.574356 99.26995) (width 0.4064) (layer "F.Cu") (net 9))
 (segment (start 160.652962 103.929613) (end 160.652962 101.270672) (width 0.4064) (layer "F.Cu") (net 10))
 (segment (start 153.867912 105.060438) (end 159.522137 105.060438) (width 0.4064) (layer "F.Cu") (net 10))
 (segment (start 159.522137 105.060438) (end 160.652962 103.929613) (width 0.4064) (layer "F.Cu") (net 10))
 (segment (start 160.652962 101.270672) (end 162.670137 99.253497) (width 0.4064) (layer "F.Cu") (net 10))
 (via (at 153.671396 105.029875) (size 0.9) (drill 0.6) (layers "F.Cu" "B.Cu") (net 10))
 (via (at 135.263346 101.130979) (size 0.9) (drill 0.6) (layers "F.Cu" "B.Cu") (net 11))
 (segment (start 157.27324 100.403985) (end 155.627612 102.049613) (width 0.4064) (layer "B.Cu") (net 11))
 (segment (start 136.18024 102.049291) (end 135.267937 101.136988) (width 0.4064) (layer "B.Cu") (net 11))
 (segment (start 157.27324 89.281844) (end 157.27324 100.403985) (width 0.4064) (layer "B.Cu") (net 11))
 (segment (start 159.061346 87.493738) (end 157.27324 89.281844) (width 0.4064) (layer "B.Cu") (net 11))
 (segment (start 155.627612 102.049613) (end 136.224965 102.049613) (width 0.4064) (layer "B.Cu") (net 11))
 (segment (start 135.267937 101.136988) (end 135.225753 101.136988) (width 0.4064) (layer "B.Cu") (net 11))
 (via (at 135.27674 103.102107) (size 0.9) (drill 0.55) (layers "F.Cu" "B.Cu") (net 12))
 (via (at 159.136503 101.98051) (size 0.9) (drill 0.6) (layers "F.Cu" "B.Cu") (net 12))
 (segment (start 135.385765 103.454) (end 157.600478 103.454) (width 0.4064) (layer "B.Cu") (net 12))
 (segment (start 157.600478 103.454) (end 158.87295 102.181529) (width 0.4064) (layer "B.Cu") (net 12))
 (segment (start 129.072465 109.020813) (end 129.072465 113.976919) (width 0.6096) (layer "F.Cu") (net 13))
 (segment (start 161.055431 120.314754) (end 161.055431 115.022638) (width 0.508) (layer "F.Cu") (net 13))
 (segment (start 161.055431 115.022638) (end 153.127462 107.094669) (width 0.508) (layer "F.Cu") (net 13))
 (segment (start 166.192746 96.367975) (end 168.172053 98.347282) (width 0.4064) (layer "F.Cu") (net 13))
 (segment (start 166.3452 106.933279) (end 152.61165 106.933279) (width 0.4064) (layer "F.Cu") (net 13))
 (segment (start 129.072465 113.976919) (end 130.321818 115.226272) (width 0.6096) (layer "F.Cu") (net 13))
 (segment (start 168.172053 105.106425) (end 166.3452 106.933279) (width 0.4064) (layer "F.Cu") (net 13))
 (segment (start 160.994081 120.376104) (end 161.055431 120.314754) (width 0.508) (layer "F.Cu") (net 13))
 (segment (start 168.172053 98.347282) (end 168.172053 105.106425) (width 0.4064) (layer "F.Cu") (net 13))
 (segment (start 165.402015 96.441504) (end 166.325718 96.441504) (width 0.4064) (layer "B.Cu") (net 13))
 (segment (start 152.875871 114.206307) (end 154.844193 112.237985) (width 0.6096) (layer "B.Cu") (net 13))
 (segment (start 162.630596 93.846197) (end 165.313959 96.52956) (width 0.4064) (layer "B.Cu") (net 13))
 (segment (start 130.573925 115.35851) (end 138.86834 115.35851) (width 0.4064) (layer "B.Cu") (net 13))
 (segment (start 138.86834 115.35851) (end 139.977528 114.249322) (width 0.4064) (layer "B.Cu") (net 13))
 (segment (start 140.004537 114.206307) (end 152.875871 114.206307) (width 0.6096) (layer "B.Cu") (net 13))
 (segment (start 165.313959 96.52956) (end 165.402015 96.441504) (width 0.4064) (layer "B.Cu") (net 13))
 (segment (start 161.489106 120.096722) (end 161.489106 120.746557) (width 0.508) (layer "B.Cu") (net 13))
 (segment (start 155.654468 114.262085) (end 161.489106 120.096722) (width 0.508) (layer "B.Cu") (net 13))
 (segment (start 162.630596 86.667379) (end 162.630596 93.846197) (width 0.4064) (layer "B.Cu") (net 13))
 (segment (start 152.559403 114.262085) (end 155.654468 114.262085) (width 0.508) (layer "B.Cu") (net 13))
 (segment (start 166.146334 96.361457) (end 166.146334 98.569988) (width 0.4064) (layer "B.Cu") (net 13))
 (segment (start 144.385115 121.706075) (end 137.745346 115.066307) (width 0.6096) (layer "B.Cu") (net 13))
 (segment (start 166.146334 98.569988) (end 163.035965 101.680357) (width 0.4064) (layer "B.Cu") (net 13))
 (segment (start 162.189862 106.050297) (end 154.580278 106.050297) (width 0.4064) (layer "F.Cu") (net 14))
 (segment (start 165.112525 93.932172) (end 164.016412 95.028285) (width 0.4064) (layer "F.Cu") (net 14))
 (segment (start 165.2492 93.935563) (end 161.003 93.935563) (width 0.4064) (layer "F.Cu") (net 14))
 (segment (start 138.661931 106.004385) (end 137.661181 107.005135) (width 0.254) (layer "F.Cu") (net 14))
 (segment (start 131.326584 104.27345) (end 131.252375 104.34766) (width 0.6096) (layer "F.Cu") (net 14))
 (segment (start 131.34389 111.990019) (end 133.041306 113.687435) (width 0.6096) (layer "F.Cu") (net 14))
 (segment (start 129.806862 104.49616) (end 129.881112 104.42191) (width 0.6096) (layer "F.Cu") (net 14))
 (segment (start 136.515965 107.18296) (end 136.697046 107.001879) (width 0.3048) (layer "F.Cu") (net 14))
 (segment (start 133.041306 115.984388) (end 131.216137 117.809557) (width 0.6096) (layer "F.Cu") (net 14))
 (segment (start 130.328081 104.404304) (end 129.79709 104.404304) (width 0.3048) (layer "F.Cu") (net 14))
 (segment (start 133.041306 113.687435) (end 133.041306 115.984388) (width 0.6096) (layer "F.Cu") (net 14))
 (segment (start 131.252375 104.34766) (end 133.776912 106.872197) (width 0.6096) (layer "F.Cu") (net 14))
 (segment (start 161.003 93.935563) (end 160.972437 93.905) (width 0.4064) (layer "F.Cu") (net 14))
 (segment (start 133.776912 106.872197) (end 136.632587 106.872197) (width 0.6096) (layer "F.Cu") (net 14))
 (segment (start 155.175843 106.024616) (end 138.588053 106.024616) (width 0.3048) (layer "F.Cu") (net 14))
 (segment (start 131.34389 104.415654) (end 131.34389 111.990019) (width 0.6096) (layer "F.Cu") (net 14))
 (segment (start 166.116712 93.932172) (end 165.112525 93.932172) (width 0.4064) (layer "F.Cu") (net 14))
 (segment (start 137.661181 107.005135) (end 136.594168 107.005135) (width 0.254) (layer "F.Cu") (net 14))
 (segment (start 164.016412 104.223747) (end 162.189862 106.050297) (width 0.4064) (layer "F.Cu") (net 14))
 (segment (start 129.881112 104.42191) (end 133.408003 104.42191) (width 0.6096) (layer "F.Cu") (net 14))
 (segment (start 130.836084 117.281094) (end 155.10034 117.281094) (width 0.508) (layer "F.Cu") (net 14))
 (segment (start 136.594168 107.005135) (end 136.415265 107.184038) (width 0.254) (layer "F.Cu") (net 14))
 (segment (start 164.016412 95.028285) (end 164.016412 104.223747) (width 0.4064) (layer "F.Cu") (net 14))
 (via (at 161.002987 93.935563) (size 0.9) (drill 0.6) (layers "F.Cu" "B.Cu") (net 14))
 (segment (start 156.363784 86.077125) (end 160.602375 86.077125) (width 0.4064) (layer "B.Cu") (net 14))
 (segment (start 161.033534 86.508285) (end 161.033534 93.813313) (width 0.4064) (layer "B.Cu") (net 14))
 (segment (start 155.626487 86.814422) (end 156.363784 86.077125) (width 0.4064) (layer "B.Cu") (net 14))
 (segment (start 160.602375 86.077125) (end 161.033534 86.508285) (width 0.4064) (layer "B.Cu") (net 14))
 (via (at 153.565481 101.112344) (size 0.9) (drill 0.6) (layers "F.Cu" "B.Cu") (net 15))
 (segment (start 155.347587 99.38115) (end 155.678481 99.38115) (width 0.4064) (layer "B.Cu") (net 15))
 (segment (start 153.641853 101.086885) (end 155.347587 99.38115) (width 0.4064) (layer "B.Cu") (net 15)))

